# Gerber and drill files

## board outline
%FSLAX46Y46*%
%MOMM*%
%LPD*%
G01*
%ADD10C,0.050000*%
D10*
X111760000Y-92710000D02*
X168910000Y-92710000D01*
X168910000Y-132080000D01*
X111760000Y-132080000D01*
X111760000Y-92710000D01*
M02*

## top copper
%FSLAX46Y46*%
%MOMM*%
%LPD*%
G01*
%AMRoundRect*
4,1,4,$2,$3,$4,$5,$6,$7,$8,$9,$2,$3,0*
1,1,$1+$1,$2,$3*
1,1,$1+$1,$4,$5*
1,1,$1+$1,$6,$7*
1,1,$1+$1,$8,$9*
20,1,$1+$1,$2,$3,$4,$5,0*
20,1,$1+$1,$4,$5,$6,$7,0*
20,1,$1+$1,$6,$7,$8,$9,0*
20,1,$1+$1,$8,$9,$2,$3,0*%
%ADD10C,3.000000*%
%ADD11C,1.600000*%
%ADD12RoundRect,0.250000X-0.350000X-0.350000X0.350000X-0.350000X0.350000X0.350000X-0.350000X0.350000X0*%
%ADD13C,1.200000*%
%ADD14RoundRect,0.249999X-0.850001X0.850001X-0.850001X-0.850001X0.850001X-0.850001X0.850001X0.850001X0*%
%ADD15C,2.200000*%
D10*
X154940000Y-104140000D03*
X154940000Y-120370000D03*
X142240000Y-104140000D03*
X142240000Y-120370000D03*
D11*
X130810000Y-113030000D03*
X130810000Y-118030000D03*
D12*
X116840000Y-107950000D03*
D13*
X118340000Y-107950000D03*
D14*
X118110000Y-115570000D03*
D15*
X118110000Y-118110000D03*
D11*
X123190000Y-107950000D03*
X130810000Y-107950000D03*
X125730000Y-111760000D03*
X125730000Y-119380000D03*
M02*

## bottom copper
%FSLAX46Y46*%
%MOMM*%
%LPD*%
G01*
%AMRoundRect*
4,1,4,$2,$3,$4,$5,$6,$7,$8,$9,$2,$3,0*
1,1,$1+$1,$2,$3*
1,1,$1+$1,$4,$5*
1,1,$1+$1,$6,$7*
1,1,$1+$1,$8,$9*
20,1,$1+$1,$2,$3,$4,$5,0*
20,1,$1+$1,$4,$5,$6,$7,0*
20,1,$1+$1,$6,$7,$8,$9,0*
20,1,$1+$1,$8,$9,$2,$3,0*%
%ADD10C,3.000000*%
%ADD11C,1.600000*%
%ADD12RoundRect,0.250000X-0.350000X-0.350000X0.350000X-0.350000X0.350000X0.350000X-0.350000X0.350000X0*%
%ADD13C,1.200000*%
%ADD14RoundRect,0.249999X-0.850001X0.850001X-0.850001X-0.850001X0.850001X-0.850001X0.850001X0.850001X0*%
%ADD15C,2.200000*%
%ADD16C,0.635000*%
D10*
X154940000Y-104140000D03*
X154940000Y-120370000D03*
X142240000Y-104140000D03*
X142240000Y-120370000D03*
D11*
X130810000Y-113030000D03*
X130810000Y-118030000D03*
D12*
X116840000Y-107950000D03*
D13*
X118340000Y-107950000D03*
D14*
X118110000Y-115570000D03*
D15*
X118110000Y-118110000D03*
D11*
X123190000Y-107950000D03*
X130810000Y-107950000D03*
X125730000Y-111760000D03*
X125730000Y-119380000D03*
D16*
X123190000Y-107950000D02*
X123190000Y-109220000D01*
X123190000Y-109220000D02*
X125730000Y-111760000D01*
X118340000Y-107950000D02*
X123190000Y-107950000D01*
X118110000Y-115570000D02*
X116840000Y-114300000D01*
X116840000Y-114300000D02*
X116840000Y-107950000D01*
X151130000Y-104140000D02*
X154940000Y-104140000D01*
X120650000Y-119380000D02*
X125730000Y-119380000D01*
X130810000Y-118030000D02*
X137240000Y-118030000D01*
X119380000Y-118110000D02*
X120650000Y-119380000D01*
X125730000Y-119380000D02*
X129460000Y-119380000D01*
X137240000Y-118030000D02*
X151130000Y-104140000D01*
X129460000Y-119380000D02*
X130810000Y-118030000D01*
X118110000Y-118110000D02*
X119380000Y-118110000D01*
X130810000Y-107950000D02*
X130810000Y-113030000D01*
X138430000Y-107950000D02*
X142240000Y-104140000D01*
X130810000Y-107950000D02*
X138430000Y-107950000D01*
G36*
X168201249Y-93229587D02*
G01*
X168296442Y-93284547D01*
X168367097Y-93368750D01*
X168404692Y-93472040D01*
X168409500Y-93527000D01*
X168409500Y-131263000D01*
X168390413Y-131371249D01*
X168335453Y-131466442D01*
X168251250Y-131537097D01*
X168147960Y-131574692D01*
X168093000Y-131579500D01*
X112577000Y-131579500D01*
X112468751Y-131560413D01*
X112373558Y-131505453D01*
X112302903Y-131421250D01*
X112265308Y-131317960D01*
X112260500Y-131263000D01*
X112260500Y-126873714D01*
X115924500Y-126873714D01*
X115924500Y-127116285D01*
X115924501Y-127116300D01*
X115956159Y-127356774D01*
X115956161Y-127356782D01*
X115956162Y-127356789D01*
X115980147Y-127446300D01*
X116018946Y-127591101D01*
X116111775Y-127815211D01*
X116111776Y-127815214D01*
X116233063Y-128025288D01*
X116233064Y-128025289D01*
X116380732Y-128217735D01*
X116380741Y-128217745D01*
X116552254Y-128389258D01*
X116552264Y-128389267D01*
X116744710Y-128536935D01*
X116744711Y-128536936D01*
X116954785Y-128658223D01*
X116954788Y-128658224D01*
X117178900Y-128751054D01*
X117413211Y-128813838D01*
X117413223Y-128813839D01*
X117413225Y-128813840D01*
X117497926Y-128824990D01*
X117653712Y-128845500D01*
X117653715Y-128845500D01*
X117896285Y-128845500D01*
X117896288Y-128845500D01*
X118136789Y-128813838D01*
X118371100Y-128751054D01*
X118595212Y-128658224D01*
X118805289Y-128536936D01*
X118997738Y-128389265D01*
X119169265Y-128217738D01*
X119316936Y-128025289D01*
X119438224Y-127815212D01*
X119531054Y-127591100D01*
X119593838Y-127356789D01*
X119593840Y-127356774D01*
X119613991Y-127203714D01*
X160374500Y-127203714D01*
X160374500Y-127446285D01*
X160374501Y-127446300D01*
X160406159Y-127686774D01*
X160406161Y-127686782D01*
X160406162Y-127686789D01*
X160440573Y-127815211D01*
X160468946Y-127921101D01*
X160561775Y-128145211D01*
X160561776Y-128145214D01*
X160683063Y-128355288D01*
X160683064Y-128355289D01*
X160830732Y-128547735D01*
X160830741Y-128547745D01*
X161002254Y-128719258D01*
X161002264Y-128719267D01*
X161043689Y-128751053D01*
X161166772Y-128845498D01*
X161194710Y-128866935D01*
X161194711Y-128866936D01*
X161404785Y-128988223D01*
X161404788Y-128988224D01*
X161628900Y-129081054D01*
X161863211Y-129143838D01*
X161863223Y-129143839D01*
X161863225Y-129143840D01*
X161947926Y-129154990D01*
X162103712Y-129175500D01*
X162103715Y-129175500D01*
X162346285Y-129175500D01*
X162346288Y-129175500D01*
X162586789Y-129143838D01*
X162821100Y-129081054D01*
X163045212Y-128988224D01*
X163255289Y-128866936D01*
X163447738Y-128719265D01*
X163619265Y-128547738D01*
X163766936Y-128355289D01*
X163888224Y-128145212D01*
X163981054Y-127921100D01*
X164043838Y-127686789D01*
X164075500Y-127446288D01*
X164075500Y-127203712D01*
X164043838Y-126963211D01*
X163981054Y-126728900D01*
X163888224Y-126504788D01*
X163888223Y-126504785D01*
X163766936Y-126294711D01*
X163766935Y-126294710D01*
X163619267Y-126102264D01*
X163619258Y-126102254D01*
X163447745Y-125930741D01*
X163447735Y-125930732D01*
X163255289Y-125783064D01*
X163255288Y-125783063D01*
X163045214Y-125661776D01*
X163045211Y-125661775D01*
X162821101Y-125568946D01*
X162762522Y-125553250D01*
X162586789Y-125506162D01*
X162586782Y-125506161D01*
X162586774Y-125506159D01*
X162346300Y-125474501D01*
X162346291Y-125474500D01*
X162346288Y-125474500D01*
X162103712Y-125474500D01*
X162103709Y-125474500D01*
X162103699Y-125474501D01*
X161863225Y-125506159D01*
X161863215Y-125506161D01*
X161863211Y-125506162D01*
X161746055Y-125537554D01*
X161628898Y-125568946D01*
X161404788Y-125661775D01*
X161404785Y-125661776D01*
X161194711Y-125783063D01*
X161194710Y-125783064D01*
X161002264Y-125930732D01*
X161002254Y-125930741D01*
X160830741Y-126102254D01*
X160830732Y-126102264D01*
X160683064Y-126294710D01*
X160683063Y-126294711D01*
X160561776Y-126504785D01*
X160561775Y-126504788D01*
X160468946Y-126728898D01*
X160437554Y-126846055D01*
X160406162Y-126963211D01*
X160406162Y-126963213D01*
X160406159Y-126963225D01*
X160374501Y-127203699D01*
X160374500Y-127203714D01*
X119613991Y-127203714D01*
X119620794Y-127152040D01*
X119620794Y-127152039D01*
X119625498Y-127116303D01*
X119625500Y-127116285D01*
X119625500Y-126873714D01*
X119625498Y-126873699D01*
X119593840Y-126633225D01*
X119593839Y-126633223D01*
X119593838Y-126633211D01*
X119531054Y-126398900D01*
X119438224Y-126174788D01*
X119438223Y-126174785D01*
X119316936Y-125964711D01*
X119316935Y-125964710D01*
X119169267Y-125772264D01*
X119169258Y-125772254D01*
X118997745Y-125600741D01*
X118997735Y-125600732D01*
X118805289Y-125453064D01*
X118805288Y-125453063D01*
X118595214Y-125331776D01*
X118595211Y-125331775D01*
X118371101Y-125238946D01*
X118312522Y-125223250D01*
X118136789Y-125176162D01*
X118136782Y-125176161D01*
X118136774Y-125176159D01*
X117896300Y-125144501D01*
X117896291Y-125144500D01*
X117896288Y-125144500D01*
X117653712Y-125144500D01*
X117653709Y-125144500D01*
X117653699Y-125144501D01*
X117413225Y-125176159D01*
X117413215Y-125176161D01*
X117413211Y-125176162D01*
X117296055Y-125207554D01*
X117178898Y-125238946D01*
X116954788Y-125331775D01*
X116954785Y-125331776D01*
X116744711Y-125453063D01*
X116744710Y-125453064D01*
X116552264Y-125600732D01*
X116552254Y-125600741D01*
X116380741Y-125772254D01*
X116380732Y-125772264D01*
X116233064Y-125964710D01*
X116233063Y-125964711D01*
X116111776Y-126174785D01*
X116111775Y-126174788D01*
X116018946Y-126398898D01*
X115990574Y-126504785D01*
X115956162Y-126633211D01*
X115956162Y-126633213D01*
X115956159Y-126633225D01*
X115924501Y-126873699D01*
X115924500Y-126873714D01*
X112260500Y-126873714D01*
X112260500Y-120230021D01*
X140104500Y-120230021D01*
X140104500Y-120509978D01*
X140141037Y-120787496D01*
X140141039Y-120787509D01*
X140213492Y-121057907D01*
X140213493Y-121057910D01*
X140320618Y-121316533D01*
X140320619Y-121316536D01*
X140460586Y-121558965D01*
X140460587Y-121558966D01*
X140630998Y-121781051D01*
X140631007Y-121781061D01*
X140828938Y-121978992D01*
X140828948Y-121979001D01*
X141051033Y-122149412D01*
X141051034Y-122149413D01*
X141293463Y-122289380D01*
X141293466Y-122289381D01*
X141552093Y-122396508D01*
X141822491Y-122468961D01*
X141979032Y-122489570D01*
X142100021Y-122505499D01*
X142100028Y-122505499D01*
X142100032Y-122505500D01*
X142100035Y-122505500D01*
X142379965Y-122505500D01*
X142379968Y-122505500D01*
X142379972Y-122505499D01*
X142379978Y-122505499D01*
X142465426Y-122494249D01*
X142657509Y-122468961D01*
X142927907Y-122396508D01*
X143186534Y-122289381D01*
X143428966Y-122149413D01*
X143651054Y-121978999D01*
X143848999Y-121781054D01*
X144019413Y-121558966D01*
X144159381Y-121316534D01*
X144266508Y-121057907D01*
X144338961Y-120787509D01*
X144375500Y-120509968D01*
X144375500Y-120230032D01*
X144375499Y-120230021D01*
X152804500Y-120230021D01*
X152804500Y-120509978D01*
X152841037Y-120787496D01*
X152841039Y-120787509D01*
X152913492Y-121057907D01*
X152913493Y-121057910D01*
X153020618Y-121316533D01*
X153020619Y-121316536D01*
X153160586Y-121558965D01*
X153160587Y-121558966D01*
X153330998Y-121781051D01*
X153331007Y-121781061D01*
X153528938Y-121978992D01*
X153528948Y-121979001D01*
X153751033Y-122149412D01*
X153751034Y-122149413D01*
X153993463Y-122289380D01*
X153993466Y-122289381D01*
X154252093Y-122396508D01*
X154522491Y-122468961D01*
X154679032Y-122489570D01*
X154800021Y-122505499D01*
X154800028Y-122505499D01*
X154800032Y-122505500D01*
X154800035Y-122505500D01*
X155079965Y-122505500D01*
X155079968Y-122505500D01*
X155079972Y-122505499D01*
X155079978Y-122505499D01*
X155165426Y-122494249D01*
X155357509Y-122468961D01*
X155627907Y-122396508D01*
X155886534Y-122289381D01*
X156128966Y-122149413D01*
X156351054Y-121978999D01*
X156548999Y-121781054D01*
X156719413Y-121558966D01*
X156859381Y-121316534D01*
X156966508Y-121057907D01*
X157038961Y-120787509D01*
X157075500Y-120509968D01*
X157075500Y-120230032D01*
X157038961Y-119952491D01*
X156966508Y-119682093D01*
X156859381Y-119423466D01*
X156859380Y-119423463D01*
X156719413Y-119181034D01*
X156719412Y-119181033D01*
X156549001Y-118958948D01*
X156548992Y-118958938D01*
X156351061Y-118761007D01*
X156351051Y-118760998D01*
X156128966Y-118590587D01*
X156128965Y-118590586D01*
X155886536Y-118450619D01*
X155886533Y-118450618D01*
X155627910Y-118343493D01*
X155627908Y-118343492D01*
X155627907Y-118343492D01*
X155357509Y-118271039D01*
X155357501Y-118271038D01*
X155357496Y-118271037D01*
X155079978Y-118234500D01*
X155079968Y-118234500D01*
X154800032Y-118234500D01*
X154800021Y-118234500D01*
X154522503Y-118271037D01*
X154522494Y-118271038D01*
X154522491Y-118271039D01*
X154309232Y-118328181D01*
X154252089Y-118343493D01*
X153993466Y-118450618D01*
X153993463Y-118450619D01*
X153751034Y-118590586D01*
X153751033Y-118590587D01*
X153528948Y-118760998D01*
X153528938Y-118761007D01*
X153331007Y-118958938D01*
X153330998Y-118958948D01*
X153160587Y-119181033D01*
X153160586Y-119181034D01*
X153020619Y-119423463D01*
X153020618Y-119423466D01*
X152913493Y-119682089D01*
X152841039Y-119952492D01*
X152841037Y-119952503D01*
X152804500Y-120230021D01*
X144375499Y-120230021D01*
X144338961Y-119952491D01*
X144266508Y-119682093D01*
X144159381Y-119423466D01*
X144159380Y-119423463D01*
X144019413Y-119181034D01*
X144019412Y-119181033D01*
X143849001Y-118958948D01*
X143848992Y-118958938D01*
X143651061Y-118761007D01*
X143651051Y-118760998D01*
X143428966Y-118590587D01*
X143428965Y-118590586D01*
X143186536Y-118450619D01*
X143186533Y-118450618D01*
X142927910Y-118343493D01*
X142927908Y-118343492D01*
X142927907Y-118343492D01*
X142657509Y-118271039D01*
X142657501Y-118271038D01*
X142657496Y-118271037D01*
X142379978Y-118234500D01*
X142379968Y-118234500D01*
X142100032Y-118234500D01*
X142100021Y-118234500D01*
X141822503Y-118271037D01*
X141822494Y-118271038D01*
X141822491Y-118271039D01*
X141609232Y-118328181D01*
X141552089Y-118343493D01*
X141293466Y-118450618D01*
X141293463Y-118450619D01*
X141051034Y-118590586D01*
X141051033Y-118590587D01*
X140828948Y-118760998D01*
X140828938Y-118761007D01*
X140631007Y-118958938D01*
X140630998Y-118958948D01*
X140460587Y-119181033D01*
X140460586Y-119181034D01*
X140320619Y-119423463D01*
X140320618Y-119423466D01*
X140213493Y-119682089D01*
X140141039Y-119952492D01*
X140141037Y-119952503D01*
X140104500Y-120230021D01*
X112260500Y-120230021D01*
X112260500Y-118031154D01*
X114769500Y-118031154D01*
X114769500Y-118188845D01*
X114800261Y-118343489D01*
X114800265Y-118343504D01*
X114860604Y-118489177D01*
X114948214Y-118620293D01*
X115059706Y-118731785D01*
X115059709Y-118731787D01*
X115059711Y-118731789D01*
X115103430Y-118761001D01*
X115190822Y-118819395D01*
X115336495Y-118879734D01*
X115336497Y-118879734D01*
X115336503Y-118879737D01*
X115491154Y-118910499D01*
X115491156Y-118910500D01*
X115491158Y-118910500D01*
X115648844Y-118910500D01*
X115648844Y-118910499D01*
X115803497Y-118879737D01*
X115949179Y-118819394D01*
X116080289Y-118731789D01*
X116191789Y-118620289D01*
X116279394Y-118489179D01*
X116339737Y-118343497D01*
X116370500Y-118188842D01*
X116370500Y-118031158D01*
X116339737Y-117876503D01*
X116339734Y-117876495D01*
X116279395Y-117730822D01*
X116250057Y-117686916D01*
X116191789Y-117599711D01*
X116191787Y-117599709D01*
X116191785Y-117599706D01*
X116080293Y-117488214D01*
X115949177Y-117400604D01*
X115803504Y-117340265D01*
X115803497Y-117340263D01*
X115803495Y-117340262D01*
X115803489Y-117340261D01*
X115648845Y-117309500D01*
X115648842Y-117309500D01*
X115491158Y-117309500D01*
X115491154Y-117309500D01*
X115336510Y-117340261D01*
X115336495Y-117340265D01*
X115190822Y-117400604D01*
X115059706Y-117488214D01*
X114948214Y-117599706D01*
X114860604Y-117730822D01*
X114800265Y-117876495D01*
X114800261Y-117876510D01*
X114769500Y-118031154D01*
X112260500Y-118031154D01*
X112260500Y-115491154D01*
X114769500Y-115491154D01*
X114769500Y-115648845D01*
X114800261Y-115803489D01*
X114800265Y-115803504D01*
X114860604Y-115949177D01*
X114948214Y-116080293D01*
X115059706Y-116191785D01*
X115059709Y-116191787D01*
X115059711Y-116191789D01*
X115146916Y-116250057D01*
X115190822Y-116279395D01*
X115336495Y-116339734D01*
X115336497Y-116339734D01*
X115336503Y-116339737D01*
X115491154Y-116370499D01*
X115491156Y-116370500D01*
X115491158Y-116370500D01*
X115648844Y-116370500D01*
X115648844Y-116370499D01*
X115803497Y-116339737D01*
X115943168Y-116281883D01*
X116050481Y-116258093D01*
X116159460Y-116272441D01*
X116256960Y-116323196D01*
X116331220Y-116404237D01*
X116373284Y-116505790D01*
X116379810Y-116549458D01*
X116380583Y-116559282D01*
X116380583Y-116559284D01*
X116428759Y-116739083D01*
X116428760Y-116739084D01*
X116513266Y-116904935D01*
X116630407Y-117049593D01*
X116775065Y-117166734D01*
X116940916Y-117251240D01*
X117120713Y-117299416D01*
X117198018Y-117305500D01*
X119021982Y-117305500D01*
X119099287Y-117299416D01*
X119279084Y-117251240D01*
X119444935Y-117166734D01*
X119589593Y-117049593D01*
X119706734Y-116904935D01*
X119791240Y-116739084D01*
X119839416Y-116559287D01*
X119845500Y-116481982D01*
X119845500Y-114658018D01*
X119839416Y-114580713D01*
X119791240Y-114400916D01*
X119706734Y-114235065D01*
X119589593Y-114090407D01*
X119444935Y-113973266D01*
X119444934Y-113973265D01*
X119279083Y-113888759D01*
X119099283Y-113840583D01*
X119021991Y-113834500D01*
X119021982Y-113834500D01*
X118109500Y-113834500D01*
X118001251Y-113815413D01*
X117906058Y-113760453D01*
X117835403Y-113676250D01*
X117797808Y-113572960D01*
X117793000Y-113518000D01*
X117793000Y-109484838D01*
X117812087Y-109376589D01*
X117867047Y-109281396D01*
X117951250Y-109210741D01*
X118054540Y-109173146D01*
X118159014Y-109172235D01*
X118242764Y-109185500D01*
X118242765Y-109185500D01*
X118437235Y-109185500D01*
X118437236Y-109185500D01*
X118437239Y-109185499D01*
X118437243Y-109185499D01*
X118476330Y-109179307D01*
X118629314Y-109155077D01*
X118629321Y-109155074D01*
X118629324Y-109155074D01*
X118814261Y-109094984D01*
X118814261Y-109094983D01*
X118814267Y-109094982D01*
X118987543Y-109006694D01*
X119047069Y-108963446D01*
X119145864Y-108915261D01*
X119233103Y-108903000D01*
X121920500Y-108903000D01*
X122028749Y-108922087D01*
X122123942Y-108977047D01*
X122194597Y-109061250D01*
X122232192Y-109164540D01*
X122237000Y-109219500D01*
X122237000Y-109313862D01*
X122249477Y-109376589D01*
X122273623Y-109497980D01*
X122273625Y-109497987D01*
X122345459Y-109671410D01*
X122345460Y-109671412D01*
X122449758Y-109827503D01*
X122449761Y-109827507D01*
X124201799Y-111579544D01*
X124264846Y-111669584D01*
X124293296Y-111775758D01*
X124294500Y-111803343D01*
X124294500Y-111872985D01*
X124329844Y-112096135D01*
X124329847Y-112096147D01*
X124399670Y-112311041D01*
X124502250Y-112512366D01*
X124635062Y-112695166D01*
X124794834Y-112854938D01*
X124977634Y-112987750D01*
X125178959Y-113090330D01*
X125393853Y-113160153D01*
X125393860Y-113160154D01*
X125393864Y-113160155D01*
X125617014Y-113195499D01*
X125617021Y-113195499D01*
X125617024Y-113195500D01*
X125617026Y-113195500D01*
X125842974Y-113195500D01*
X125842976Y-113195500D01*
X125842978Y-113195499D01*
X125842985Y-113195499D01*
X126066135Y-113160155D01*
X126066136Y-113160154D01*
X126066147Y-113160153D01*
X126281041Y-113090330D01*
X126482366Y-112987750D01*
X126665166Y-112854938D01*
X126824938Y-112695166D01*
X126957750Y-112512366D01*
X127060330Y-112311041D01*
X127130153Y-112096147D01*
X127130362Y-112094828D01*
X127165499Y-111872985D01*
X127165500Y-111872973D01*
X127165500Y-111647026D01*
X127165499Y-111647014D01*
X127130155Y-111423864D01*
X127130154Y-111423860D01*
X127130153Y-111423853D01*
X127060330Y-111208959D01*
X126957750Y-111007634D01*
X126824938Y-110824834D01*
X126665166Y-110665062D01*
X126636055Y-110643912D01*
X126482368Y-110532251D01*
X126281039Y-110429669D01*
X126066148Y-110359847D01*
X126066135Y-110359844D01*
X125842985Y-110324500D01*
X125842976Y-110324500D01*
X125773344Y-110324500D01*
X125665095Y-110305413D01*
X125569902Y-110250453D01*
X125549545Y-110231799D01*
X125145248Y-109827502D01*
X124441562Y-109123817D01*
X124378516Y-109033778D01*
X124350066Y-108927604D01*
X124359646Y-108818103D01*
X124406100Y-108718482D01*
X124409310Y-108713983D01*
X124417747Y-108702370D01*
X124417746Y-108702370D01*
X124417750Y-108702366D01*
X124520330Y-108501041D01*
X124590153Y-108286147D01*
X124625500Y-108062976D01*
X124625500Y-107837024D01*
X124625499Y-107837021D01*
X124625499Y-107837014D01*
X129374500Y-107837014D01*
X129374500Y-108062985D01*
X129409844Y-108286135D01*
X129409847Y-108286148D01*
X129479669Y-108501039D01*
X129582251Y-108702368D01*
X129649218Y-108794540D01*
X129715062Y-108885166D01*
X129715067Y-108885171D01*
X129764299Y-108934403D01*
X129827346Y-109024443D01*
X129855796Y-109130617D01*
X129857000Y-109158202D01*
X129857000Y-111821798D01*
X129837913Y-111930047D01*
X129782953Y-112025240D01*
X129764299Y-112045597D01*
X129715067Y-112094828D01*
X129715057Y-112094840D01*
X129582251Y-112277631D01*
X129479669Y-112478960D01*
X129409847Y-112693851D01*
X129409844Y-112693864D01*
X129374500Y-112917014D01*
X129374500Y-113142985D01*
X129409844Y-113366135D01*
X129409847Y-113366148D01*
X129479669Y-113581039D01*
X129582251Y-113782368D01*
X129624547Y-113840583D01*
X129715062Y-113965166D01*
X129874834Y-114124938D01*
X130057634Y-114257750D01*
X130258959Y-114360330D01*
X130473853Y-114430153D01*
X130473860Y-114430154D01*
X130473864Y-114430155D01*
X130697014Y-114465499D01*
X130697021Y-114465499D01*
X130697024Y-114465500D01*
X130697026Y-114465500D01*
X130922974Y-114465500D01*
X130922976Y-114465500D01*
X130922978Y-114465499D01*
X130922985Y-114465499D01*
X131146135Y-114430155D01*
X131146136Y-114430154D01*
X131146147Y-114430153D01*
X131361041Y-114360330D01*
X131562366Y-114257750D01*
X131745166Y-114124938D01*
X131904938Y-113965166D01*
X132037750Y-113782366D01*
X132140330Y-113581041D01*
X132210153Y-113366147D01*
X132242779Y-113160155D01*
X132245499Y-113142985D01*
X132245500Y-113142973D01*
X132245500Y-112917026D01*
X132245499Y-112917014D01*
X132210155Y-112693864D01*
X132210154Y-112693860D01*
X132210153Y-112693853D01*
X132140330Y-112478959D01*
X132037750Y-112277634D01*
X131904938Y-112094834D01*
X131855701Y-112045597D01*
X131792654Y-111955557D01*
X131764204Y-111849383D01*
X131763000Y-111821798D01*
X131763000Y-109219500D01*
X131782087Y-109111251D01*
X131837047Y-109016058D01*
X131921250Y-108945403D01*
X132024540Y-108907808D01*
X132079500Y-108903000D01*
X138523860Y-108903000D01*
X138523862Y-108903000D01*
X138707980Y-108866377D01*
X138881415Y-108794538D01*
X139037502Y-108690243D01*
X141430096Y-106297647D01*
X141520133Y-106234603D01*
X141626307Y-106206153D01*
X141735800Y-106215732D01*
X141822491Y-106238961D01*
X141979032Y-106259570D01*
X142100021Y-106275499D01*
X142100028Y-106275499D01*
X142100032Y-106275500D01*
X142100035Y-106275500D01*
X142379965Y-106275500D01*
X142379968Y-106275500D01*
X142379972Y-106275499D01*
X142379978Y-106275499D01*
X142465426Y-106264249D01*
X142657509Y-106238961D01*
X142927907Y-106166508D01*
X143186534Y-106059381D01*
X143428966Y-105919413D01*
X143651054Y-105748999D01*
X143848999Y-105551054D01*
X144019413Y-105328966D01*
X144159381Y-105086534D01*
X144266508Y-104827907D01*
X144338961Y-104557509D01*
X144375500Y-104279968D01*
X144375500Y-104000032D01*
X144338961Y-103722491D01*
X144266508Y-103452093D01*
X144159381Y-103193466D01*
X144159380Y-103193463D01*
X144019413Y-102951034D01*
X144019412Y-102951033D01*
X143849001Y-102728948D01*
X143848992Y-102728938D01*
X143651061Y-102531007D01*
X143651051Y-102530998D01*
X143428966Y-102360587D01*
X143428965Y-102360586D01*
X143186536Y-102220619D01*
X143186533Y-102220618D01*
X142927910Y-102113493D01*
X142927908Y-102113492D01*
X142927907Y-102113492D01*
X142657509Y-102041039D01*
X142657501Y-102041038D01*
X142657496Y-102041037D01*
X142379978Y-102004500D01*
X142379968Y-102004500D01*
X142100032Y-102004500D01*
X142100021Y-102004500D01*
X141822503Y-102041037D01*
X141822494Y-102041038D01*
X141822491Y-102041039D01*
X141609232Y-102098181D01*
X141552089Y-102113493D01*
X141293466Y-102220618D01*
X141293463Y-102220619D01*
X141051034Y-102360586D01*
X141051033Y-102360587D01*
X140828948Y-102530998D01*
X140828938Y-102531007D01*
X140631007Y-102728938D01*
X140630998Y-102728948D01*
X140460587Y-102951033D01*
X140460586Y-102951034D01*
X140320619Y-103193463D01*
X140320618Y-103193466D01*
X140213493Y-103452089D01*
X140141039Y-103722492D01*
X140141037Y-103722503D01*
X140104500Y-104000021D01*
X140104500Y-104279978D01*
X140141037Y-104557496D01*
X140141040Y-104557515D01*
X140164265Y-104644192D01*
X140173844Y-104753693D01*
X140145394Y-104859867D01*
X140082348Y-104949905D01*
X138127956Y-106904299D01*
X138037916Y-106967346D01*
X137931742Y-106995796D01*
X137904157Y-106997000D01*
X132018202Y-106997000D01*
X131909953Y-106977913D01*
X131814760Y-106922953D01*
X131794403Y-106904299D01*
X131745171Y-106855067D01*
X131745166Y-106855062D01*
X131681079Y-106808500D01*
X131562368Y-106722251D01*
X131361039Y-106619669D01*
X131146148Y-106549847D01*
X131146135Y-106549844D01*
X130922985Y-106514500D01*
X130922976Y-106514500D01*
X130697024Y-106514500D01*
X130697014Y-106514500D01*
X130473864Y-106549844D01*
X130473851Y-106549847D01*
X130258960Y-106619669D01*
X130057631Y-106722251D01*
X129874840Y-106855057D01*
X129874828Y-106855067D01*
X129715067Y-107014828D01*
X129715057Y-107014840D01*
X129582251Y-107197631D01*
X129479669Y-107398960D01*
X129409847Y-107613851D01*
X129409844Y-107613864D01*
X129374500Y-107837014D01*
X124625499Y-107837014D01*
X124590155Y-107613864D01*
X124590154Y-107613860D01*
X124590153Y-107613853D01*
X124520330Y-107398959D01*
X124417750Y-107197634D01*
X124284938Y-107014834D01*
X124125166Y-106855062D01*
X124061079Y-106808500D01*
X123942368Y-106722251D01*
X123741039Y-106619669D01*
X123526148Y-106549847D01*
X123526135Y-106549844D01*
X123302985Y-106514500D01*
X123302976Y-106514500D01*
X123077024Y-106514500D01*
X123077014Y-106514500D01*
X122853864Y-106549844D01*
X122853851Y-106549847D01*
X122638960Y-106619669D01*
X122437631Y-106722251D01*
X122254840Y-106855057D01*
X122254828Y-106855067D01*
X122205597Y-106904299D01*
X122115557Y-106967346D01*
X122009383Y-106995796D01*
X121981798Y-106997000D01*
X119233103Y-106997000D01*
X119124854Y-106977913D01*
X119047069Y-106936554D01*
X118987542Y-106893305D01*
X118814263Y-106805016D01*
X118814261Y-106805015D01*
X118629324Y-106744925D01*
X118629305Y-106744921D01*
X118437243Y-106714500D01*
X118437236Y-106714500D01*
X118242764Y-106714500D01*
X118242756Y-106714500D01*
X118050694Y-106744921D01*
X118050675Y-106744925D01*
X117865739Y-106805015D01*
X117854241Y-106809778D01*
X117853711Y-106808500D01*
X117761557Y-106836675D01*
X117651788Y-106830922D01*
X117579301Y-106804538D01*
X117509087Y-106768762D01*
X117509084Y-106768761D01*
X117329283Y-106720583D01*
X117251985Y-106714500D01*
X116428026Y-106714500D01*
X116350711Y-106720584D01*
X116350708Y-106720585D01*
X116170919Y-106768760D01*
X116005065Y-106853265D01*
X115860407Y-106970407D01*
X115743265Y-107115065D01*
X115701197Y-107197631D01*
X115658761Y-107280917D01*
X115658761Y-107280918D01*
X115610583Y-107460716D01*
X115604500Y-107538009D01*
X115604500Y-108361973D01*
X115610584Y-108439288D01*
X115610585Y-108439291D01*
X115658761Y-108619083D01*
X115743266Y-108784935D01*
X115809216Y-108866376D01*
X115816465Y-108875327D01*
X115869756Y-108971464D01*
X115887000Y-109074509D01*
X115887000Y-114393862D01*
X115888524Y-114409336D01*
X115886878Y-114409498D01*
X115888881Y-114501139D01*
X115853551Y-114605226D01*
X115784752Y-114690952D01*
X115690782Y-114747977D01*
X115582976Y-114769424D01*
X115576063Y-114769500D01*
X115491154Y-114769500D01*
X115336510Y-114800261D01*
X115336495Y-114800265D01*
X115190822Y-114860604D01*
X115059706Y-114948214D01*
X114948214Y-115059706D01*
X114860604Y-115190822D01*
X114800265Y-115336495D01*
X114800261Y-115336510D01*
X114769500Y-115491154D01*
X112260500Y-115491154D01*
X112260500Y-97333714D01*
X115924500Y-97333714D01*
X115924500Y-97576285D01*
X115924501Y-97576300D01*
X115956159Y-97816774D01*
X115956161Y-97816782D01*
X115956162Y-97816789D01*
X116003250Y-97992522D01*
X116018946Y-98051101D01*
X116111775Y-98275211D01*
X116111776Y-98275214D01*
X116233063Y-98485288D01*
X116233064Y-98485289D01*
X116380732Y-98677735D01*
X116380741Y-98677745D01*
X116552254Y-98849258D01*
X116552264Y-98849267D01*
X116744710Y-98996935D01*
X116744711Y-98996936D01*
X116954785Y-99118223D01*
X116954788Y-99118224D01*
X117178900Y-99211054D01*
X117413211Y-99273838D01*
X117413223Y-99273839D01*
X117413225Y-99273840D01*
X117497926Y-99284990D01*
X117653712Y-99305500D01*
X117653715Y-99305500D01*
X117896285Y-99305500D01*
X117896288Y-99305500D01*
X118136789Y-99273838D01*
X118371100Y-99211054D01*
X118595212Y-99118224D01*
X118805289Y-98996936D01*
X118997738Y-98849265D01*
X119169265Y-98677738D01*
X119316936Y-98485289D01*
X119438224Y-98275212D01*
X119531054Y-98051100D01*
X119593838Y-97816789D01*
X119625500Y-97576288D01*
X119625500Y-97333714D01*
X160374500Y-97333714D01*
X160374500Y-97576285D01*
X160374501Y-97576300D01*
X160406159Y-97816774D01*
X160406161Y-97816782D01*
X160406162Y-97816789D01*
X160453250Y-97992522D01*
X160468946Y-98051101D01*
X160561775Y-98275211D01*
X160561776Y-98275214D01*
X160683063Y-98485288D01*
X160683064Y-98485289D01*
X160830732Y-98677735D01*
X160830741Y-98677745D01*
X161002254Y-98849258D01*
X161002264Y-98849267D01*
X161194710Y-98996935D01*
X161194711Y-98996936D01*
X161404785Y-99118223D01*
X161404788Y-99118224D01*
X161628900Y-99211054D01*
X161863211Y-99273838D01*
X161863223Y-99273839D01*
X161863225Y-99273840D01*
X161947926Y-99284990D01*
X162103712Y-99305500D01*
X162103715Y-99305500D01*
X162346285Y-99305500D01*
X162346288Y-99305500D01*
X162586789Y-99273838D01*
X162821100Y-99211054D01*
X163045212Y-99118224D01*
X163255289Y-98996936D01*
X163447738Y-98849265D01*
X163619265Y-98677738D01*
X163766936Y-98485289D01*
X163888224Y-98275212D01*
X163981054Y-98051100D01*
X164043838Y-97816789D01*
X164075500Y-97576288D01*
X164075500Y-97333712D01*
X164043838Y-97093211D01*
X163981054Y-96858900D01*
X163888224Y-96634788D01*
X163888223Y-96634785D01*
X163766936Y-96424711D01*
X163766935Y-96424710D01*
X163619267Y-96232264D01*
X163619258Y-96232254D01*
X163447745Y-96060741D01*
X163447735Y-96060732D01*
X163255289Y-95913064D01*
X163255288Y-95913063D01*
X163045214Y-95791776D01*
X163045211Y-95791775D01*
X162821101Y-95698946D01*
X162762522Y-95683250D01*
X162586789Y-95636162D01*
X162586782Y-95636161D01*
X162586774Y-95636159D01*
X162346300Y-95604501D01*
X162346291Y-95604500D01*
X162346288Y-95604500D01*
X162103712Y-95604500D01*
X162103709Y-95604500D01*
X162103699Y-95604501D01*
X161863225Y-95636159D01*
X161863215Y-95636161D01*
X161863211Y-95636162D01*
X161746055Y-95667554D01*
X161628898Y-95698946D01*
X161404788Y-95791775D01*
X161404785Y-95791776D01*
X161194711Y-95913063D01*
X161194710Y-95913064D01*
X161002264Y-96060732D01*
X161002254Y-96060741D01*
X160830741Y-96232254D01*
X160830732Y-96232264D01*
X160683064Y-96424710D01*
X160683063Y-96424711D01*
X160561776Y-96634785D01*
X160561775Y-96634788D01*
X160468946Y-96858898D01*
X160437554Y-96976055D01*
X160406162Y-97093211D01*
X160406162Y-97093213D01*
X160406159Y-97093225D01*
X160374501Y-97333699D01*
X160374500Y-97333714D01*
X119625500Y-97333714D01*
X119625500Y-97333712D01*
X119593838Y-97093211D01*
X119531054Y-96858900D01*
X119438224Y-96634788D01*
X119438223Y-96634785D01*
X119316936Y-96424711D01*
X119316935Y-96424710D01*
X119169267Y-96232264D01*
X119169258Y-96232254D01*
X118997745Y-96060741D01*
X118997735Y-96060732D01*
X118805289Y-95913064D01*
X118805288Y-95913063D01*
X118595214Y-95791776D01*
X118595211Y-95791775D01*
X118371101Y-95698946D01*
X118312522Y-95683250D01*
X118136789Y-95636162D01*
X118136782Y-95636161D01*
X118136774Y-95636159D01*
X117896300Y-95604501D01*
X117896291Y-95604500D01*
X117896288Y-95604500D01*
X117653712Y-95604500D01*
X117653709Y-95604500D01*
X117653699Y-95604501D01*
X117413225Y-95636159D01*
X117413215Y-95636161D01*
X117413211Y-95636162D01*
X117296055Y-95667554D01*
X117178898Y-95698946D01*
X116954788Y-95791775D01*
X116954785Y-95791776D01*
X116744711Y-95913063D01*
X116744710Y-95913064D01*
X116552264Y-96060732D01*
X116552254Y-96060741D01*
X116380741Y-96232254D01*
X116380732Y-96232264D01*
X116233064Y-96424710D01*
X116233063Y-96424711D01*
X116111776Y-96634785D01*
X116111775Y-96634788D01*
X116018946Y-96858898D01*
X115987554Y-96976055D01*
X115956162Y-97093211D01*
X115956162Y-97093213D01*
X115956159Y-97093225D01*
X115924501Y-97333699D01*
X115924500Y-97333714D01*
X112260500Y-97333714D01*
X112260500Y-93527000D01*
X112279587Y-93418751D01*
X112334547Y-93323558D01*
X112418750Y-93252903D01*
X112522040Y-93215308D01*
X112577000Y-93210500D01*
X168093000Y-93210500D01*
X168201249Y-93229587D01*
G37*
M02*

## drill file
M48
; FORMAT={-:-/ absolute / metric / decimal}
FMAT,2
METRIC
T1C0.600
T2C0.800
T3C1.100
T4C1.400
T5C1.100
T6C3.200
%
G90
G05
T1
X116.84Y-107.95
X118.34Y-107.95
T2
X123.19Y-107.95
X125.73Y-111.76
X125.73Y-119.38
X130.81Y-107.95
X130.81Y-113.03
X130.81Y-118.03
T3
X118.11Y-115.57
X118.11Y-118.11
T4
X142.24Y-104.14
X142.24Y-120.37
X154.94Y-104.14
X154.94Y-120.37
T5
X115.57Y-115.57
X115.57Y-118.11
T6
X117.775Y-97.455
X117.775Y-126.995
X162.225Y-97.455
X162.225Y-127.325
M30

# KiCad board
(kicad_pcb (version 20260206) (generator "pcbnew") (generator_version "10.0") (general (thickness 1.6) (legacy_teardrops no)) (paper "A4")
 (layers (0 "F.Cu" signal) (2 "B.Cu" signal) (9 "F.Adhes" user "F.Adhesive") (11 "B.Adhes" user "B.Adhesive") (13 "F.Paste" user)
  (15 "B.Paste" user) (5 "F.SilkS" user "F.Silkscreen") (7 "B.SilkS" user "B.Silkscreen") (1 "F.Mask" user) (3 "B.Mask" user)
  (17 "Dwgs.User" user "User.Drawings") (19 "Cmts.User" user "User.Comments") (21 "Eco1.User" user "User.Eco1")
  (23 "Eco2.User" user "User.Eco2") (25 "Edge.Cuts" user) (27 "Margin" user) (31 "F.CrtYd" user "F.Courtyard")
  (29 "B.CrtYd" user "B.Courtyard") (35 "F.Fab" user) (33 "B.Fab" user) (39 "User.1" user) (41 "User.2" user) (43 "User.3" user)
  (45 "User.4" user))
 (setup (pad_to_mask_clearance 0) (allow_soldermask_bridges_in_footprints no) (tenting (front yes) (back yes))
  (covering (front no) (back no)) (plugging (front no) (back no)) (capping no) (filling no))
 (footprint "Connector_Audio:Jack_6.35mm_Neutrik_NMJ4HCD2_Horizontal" (layer "F.Cu") (at 142.24 104.14)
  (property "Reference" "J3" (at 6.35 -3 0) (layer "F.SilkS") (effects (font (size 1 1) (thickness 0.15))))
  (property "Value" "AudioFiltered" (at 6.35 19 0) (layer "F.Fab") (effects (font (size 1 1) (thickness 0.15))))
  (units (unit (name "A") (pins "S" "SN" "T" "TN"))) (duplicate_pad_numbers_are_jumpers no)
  (pad "S" thru_hole circle (at 12.7 0) (size 3 3) (drill 1.4) (layers "*.Cu" "*.Mask") (remove_unused_layers no) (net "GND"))
  (pad "SN" thru_hole circle (at 12.7 16.23) (size 3 3) (drill 1.4) (layers "*.Cu" "*.Mask") (remove_unused_layers no)
   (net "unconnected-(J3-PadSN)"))
  (pad "T" thru_hole circle (at 0 0) (size 3 3) (drill 1.4) (layers "*.Cu" "*.Mask") (remove_unused_layers no) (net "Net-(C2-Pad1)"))
  (pad "TN" thru_hole circle (at 0 16.23) (size 3 3) (drill 1.4) (layers "*.Cu" "*.Mask") (remove_unused_layers no)
   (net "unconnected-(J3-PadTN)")))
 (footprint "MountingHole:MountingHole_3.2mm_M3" (layer "F.Cu") (at 117.775 126.995)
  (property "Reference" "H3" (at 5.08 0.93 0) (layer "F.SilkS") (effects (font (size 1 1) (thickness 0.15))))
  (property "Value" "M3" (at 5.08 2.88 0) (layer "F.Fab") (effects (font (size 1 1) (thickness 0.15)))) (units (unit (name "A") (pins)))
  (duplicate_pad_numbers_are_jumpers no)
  (pad "" np_thru_hole circle (at 0 0) (size 3.2 3.2) (drill 3.2) (layers "*.Cu" "*.Mask")))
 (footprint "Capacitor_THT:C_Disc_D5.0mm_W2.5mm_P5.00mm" (layer "F.Cu") (at 130.81 113.03 -90)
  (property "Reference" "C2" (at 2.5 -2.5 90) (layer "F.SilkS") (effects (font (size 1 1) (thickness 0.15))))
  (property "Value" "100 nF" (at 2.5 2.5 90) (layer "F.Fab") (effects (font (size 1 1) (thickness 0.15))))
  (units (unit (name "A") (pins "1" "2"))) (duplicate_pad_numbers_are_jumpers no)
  (pad "1" thru_hole circle (at 0 0 270) (size 1.6 1.6) (drill 0.8) (layers "*.Cu" "*.Mask") (remove_unused_layers no) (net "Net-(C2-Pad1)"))
  (pad "2" thru_hole circle (at 5 0 270) (size 1.6 1.6) (drill 0.8) (layers "*.Cu" "*.Mask") (remove_unused_layers no) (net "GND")))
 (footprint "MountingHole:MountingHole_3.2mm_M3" (layer "F.Cu") (at 162.225 127.325)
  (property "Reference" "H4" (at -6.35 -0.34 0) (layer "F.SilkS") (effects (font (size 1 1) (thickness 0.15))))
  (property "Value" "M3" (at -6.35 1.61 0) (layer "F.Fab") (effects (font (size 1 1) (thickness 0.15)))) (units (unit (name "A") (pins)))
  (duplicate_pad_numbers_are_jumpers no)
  (pad "" np_thru_hole circle (at 0 0) (size 3.2 3.2) (drill 3.2) (layers "*.Cu" "*.Mask")))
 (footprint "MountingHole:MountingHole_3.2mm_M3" (layer "F.Cu") (at 162.225 97.455)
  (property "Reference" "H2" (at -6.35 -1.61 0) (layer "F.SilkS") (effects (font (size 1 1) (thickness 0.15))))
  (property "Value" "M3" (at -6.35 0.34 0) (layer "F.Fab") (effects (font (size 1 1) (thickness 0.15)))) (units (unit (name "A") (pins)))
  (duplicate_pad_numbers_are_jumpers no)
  (pad "" np_thru_hole circle (at 0 0) (size 3.2 3.2) (drill 3.2) (layers "*.Cu" "*.Mask")))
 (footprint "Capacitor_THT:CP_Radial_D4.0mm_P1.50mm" (layer "F.Cu") (at 116.84 107.95)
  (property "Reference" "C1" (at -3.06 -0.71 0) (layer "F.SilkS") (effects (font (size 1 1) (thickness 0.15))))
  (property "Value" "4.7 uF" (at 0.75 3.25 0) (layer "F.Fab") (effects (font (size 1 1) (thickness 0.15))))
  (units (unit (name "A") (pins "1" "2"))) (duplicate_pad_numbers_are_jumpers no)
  (pad "1" thru_hole roundrect (at 0 0) (size 1.2 1.2) (drill 0.6) (layers "*.Cu" "*.Mask") (remove_unused_layers no)
   (roundrect_rratio 0.208333) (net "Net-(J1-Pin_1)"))
  (pad "2" thru_hole circle (at 1.5 0) (size 1.2 1.2) (drill 0.6) (layers "*.Cu" "*.Mask") (remove_unused_layers no) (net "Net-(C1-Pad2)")))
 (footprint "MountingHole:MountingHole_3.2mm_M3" (layer "F.Cu") (at 117.775 97.455)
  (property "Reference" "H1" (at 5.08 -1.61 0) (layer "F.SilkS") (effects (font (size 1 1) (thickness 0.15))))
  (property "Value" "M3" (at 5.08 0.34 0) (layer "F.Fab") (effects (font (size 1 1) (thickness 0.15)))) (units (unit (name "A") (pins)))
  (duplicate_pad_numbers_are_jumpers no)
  (pad "" np_thru_hole circle (at 0 0) (size 3.2 3.2) (drill 3.2) (layers "*.Cu" "*.Mask")))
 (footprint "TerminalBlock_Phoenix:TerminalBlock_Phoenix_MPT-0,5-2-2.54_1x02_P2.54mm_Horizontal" (layer "F.Cu") (at 118.11 115.57 -90)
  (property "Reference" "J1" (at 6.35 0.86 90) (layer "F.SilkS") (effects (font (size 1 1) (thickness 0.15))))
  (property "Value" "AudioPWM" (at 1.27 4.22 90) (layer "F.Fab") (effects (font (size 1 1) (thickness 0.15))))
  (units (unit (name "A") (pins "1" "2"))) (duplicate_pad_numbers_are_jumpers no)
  (pad "" np_thru_hole circle (at 0 2.54 270) (size 1.1 1.1) (drill 1.1) (layers "*.Cu" "*.Mask"))
  (pad "" np_thru_hole circle (at 2.54 2.54 270) (size 1.1 1.1) (drill 1.1) (layers "*.Cu" "*.Mask"))
  (pad "1" thru_hole roundrect (at 0 0 270) (size 2.2 2.2) (drill 1.1) (layers "*.Cu" "*.Mask") (remove_unused_layers no)
   (roundrect_rratio 0.113636) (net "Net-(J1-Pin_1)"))
  (pad "2" thru_hole circle (at 2.54 0 270) (size 2.2 2.2) (drill 1.1) (layers "*.Cu" "*.Mask") (remove_unused_layers no) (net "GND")))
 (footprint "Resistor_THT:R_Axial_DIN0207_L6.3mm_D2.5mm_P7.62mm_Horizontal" (layer "F.Cu") (at 123.19 107.95)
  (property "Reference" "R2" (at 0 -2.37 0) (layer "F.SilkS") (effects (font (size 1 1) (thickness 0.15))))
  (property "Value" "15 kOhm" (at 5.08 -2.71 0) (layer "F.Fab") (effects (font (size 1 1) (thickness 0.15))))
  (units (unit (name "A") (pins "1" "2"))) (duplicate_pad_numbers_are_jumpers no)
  (pad "1" thru_hole circle (at 0 0) (size 1.6 1.6) (drill 0.8) (layers "*.Cu" "*.Mask") (remove_unused_layers no) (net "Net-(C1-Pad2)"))
  (pad "2" thru_hole circle (at 7.62 0) (size 1.6 1.6) (drill 0.8) (layers "*.Cu" "*.Mask") (remove_unused_layers no) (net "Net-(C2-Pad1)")))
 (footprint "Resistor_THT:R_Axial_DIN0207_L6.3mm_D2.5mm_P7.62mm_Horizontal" (layer "F.Cu") (at 125.73 111.76 -90)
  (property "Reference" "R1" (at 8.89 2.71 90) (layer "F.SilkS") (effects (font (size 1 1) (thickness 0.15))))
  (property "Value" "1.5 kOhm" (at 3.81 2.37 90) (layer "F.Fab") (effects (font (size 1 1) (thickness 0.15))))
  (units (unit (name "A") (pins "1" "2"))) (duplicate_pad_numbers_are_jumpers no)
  (pad "1" thru_hole circle (at 0 0 270) (size 1.6 1.6) (drill 0.8) (layers "*.Cu" "*.Mask") (remove_unused_layers no) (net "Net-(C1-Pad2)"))
  (pad "2" thru_hole circle (at 7.62 0 270) (size 1.6 1.6) (drill 0.8) (layers "*.Cu" "*.Mask") (remove_unused_layers no) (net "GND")))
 (gr_rect (start 111.76 92.71) (end 168.91 132.08) (stroke (width 0.05) (type default)) (fill no) (layer "Edge.Cuts"))
 (segment (start 123.19 107.95) (end 123.19 109.22) (width 0.635) (layer "B.Cu") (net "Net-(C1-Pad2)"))
 (segment (start 123.19 109.22) (end 125.73 111.76) (width 0.635) (layer "B.Cu") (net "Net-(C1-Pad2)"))
 (segment (start 118.34 107.95) (end 123.19 107.95) (width 0.635) (layer "B.Cu") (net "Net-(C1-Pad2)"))
 (segment (start 118.11 115.57) (end 116.84 114.3) (width 0.635) (layer "B.Cu") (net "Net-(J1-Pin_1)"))
 (segment (start 116.84 114.3) (end 116.84 107.95) (width 0.635) (layer "B.Cu") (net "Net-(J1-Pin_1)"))
 (segment (start 151.13 104.14) (end 154.94 104.14) (width 0.635) (layer "B.Cu") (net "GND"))
 (segment (start 120.65 119.38) (end 125.73 119.38) (width 0.635) (layer "B.Cu") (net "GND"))
 (segment (start 130.81 118.03) (end 137.24 118.03) (width 0.635) (layer "B.Cu") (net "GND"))
 (segment (start 119.38 118.11) (end 120.65 119.38) (width 0.635) (layer "B.Cu") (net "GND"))
 (segment (start 125.73 119.38) (end 129.46 119.38) (width 0.635) (layer "B.Cu") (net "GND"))
 (segment (start 137.24 118.03) (end 151.13 104.14) (width 0.635) (layer "B.Cu") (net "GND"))
 (segment (start 129.46 119.38) (end 130.81 118.03) (width 0.635) (layer "B.Cu") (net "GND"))
 (segment (start 118.11 118.11) (end 119.38 118.11) (width 0.635) (layer "B.Cu") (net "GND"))
 (segment (start 130.81 107.95) (end 130.81 113.03) (width 0.635) (layer "B.Cu") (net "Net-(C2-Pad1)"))
 (segment (start 138.43 107.95) (end 142.24 104.14) (width 0.635) (layer "B.Cu") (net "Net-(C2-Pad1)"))
 (segment (start 130.81 107.95) (end 138.43 107.95) (width 0.635) (layer "B.Cu") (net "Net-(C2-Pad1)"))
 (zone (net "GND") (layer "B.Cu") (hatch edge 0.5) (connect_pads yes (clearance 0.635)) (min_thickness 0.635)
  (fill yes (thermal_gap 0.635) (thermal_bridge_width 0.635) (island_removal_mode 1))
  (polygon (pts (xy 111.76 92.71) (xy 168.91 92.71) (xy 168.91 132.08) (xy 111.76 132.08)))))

